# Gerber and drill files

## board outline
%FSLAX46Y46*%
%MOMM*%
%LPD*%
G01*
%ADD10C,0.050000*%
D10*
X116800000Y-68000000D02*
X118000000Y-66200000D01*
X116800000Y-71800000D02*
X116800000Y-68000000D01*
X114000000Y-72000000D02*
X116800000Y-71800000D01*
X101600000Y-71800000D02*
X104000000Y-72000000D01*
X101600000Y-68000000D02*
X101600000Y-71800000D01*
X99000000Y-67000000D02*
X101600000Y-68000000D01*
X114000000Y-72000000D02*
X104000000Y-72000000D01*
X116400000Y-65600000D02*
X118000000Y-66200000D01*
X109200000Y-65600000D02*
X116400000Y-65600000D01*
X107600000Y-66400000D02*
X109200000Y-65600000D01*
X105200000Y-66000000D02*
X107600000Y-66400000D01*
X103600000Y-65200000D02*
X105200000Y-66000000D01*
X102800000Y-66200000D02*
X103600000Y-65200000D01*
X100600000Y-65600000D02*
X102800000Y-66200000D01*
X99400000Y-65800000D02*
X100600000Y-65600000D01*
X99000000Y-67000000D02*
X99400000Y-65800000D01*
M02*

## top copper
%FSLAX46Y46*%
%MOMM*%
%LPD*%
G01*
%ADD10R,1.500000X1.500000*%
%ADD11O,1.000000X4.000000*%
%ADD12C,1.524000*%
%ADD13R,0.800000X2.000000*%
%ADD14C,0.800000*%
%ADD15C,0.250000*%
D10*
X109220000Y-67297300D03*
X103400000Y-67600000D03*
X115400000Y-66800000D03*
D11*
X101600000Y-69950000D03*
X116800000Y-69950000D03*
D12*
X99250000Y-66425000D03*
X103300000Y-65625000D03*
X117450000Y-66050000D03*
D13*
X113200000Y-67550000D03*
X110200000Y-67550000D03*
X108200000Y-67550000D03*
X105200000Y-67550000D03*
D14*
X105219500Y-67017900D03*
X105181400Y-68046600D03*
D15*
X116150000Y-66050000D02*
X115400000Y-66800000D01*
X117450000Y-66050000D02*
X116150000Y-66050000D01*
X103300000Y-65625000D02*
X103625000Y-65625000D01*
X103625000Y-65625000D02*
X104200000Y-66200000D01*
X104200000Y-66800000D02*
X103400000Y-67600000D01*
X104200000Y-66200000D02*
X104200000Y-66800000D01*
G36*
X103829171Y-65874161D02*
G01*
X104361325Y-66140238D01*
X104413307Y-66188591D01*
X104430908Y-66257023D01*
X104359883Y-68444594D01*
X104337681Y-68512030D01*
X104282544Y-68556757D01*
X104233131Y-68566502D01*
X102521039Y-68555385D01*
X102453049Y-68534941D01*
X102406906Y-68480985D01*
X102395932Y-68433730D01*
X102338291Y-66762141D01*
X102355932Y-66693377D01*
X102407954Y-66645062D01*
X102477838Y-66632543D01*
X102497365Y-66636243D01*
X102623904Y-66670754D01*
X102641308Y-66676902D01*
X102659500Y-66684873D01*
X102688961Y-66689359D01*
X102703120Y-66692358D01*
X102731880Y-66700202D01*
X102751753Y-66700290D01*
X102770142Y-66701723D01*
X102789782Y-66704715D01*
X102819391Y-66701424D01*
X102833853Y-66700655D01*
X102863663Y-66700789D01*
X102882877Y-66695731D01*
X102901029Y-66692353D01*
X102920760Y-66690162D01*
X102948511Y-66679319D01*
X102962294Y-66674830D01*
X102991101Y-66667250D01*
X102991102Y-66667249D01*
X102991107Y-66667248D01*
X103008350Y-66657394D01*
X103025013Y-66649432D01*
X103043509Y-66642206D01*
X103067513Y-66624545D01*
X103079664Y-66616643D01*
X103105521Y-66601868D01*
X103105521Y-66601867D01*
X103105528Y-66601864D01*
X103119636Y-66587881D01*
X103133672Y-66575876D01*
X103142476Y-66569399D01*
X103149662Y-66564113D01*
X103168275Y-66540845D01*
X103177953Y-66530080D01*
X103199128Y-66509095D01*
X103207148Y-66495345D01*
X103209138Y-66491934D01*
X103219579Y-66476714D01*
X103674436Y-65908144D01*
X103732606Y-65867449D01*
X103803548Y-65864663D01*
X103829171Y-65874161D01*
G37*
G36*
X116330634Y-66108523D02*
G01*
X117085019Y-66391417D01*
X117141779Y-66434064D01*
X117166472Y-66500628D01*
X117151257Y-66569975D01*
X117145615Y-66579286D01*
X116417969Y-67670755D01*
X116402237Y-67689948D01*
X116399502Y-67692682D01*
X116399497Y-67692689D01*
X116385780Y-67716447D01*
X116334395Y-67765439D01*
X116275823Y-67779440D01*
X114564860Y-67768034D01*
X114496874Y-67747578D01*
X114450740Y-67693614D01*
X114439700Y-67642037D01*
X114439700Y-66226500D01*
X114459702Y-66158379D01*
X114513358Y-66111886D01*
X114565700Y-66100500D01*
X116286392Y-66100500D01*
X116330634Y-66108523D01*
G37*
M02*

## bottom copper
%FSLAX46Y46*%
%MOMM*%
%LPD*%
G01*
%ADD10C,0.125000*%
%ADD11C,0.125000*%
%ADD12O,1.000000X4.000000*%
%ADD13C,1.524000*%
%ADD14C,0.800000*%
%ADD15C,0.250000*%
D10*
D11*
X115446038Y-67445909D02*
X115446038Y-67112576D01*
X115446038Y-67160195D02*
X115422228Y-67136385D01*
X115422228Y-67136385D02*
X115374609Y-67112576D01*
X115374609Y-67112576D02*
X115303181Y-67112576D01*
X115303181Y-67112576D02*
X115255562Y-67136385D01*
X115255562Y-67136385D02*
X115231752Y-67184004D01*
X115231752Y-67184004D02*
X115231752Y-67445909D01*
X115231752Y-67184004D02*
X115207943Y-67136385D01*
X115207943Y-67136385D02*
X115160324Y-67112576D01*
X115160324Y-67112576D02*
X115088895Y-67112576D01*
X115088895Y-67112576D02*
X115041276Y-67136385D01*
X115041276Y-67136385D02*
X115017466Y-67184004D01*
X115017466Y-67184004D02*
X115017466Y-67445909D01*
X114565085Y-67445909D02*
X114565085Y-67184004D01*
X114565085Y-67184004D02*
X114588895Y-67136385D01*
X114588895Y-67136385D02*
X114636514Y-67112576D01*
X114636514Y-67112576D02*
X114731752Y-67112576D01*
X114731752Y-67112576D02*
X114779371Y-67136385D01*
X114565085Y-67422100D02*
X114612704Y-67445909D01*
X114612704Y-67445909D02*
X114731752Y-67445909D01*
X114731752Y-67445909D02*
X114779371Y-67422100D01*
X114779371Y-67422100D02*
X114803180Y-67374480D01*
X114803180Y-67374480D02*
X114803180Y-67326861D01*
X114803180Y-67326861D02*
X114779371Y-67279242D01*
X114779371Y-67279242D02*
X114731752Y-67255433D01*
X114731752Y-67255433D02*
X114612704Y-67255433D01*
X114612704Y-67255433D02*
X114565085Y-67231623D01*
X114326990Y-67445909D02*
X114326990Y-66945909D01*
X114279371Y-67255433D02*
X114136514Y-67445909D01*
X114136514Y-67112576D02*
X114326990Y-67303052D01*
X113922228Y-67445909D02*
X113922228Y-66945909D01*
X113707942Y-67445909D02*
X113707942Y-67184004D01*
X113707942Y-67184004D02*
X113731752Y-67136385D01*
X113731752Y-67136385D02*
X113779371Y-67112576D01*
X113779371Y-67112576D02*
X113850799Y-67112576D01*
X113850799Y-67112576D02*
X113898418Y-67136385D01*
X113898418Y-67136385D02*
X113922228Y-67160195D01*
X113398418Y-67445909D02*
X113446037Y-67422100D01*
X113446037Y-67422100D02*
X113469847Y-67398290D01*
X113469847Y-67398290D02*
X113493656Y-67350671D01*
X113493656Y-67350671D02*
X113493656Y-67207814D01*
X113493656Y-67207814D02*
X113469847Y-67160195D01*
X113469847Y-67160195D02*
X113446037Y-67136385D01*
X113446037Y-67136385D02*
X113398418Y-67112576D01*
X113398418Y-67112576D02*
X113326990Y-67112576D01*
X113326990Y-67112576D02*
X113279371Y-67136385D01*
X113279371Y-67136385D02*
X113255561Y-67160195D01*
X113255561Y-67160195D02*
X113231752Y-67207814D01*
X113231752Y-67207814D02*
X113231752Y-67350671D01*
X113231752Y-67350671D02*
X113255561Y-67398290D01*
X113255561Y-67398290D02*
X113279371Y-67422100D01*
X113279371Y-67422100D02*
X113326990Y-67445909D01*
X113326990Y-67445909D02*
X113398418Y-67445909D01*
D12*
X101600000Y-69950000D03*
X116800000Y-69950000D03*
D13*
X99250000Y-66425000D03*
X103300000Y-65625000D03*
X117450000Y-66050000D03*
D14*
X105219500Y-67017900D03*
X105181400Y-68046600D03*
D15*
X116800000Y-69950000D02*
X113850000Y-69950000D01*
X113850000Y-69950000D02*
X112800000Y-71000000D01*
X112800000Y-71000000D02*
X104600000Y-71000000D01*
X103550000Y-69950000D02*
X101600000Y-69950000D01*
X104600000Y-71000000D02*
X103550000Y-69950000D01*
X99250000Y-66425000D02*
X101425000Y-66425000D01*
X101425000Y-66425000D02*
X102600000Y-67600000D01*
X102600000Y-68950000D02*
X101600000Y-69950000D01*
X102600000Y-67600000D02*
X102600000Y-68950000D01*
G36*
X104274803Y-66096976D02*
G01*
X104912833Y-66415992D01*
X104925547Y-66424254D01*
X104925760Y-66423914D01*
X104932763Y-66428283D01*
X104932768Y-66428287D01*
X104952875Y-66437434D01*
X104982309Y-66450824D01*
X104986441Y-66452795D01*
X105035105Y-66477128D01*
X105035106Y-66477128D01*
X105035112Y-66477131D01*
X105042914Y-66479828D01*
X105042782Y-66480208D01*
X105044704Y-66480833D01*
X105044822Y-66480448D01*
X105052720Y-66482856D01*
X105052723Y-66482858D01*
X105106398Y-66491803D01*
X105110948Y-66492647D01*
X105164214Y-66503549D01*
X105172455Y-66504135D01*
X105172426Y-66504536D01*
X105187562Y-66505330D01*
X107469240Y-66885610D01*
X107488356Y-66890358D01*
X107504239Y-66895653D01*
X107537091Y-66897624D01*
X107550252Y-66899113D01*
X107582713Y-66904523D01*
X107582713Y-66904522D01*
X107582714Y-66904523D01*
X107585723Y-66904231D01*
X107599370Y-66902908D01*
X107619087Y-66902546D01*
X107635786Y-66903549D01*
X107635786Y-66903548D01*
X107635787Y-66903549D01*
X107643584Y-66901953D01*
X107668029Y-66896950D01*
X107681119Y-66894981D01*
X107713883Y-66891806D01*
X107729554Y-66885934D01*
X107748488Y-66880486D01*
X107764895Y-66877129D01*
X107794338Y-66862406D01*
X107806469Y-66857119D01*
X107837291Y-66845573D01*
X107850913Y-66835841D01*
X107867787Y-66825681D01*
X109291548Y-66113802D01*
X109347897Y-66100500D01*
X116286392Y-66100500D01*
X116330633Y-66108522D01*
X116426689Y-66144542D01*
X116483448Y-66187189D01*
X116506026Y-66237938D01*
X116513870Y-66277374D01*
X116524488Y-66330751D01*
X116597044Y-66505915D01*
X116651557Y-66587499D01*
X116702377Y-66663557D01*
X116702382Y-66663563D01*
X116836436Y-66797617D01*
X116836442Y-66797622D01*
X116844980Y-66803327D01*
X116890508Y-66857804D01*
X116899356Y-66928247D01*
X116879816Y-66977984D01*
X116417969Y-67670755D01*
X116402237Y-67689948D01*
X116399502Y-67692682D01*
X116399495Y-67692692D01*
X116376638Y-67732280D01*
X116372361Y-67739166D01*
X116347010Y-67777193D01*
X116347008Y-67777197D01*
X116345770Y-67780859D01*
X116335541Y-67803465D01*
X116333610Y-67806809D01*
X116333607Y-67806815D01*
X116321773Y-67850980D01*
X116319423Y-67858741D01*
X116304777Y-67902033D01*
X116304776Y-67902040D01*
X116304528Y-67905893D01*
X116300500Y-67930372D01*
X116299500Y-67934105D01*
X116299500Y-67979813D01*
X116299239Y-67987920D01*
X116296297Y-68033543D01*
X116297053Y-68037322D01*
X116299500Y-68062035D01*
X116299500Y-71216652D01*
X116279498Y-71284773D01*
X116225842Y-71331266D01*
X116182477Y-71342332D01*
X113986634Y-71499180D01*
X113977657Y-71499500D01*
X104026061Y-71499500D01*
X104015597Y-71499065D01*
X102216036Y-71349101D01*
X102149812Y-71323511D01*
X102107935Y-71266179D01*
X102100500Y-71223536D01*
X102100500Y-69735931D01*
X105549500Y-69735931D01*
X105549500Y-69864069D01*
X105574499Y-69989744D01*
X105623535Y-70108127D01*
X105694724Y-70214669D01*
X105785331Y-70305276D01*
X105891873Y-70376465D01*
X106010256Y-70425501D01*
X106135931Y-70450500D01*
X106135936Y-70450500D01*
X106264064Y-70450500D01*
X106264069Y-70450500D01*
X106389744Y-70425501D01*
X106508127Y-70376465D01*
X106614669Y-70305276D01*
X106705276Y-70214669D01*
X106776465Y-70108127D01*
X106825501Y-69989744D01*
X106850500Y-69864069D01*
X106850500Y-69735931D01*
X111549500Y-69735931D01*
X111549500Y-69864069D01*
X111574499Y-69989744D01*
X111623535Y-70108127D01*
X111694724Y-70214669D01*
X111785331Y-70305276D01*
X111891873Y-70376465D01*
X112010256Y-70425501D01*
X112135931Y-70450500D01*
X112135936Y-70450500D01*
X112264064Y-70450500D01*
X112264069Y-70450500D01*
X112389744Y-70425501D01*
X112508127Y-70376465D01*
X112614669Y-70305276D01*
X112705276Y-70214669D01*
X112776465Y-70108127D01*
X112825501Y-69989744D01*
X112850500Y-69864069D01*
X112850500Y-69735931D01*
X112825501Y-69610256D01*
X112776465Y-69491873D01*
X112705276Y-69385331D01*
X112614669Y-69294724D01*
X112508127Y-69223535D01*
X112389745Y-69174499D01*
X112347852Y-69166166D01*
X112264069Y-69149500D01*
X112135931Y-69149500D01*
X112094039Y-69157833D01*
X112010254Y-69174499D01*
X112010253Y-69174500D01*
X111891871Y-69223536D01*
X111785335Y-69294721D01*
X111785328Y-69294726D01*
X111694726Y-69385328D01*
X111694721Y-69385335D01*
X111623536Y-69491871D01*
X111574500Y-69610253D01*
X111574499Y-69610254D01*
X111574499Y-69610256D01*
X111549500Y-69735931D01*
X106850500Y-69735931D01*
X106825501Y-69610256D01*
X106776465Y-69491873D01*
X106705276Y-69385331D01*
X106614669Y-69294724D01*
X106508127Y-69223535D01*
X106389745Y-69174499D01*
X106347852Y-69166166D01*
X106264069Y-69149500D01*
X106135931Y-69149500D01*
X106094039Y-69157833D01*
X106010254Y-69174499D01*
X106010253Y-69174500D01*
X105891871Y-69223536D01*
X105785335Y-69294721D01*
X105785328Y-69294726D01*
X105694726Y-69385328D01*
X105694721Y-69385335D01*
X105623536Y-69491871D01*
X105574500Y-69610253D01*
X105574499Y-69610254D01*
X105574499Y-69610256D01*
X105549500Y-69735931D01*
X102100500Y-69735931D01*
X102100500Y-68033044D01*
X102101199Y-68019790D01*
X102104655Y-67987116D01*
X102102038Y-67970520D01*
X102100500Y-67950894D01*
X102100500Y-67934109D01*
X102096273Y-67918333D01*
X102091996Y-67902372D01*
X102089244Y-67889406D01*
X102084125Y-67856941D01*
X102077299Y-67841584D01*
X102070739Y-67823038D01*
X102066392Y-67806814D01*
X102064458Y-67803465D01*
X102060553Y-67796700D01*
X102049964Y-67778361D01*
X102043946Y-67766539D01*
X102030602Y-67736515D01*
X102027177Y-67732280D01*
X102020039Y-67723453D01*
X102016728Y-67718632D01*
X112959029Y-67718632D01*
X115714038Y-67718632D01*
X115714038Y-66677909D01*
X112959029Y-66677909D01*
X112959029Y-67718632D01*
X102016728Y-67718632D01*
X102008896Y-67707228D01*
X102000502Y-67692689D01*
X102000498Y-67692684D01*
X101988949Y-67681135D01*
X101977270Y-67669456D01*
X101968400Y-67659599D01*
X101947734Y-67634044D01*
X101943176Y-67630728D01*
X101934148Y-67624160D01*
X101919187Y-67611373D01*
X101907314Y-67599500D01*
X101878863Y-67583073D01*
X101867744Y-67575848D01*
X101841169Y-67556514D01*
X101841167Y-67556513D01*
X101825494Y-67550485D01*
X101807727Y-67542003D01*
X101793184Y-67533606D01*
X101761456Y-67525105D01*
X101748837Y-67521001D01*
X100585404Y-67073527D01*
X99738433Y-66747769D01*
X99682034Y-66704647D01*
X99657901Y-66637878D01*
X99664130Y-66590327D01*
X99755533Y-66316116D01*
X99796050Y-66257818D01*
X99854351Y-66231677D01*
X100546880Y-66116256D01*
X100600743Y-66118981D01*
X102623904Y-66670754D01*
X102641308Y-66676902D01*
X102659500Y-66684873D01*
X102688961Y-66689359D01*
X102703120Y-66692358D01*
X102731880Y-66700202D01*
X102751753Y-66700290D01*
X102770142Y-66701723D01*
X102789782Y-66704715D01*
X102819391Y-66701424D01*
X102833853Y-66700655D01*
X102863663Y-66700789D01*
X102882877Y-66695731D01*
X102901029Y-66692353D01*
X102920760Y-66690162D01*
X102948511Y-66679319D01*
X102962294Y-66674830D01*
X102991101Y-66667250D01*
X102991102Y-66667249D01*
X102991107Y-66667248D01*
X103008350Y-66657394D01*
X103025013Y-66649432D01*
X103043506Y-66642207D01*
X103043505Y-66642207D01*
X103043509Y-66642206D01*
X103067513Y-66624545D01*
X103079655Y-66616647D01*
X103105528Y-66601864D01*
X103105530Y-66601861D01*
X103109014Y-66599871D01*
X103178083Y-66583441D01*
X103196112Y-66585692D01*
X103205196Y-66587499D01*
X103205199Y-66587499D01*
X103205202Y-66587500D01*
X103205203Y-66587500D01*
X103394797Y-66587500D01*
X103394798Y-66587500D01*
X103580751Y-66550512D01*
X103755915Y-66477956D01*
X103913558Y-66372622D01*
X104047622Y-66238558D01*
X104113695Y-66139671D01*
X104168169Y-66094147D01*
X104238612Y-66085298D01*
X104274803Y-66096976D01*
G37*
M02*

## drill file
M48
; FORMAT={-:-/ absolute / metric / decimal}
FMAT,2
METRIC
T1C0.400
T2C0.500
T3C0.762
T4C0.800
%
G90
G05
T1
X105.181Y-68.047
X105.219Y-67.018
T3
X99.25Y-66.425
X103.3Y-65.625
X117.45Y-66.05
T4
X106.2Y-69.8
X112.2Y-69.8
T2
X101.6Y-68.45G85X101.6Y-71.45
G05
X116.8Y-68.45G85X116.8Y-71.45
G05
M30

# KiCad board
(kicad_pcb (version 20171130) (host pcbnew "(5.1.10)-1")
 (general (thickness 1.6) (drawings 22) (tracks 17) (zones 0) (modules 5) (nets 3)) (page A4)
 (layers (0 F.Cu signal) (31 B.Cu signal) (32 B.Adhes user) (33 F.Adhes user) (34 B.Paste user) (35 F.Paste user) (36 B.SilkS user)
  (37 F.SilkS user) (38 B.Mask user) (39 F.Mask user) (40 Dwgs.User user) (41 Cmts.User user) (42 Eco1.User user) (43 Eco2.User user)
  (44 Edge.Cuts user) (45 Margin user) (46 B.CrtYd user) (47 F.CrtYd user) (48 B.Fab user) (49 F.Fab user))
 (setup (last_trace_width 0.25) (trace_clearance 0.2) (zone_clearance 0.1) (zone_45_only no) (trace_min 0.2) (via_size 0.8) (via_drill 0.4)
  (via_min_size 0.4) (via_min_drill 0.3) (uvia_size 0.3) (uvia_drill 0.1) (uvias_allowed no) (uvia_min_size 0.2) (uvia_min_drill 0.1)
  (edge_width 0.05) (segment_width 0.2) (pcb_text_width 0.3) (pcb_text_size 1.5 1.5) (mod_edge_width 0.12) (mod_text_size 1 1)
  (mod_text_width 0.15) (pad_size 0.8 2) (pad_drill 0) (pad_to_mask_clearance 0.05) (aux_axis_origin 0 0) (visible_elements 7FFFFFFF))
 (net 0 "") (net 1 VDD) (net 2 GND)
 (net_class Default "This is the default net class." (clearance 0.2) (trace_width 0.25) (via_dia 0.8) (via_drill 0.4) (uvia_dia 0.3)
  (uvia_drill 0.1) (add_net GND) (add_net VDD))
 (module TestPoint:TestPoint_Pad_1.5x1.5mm (layer F.Cu) (at 109.22 67.2973)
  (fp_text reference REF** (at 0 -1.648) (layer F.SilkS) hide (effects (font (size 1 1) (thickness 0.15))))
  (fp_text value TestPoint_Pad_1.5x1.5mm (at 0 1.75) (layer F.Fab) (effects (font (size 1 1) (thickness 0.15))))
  (pad 1 smd rect (at 0 0) (size 1.5 1.5) (layers F.Cu F.Mask)))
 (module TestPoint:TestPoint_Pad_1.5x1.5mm (layer F.Cu) (at 103.4 67.6)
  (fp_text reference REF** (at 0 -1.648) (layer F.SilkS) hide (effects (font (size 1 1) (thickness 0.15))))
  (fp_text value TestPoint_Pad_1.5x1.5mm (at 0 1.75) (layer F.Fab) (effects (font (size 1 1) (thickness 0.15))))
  (pad 1 smd rect (at 0 0) (size 1.5 1.5) (layers F.Cu F.Mask) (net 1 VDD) (zone_connect 2)))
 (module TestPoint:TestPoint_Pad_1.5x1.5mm (layer F.Cu) (at 115.4 66.8)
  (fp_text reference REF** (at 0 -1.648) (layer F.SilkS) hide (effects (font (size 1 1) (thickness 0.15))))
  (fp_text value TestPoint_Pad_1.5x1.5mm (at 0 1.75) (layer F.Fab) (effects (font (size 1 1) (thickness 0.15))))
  (pad 1 smd rect (at 0 0) (size 1.5 1.5) (layers F.Cu F.Mask) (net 1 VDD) (zone_connect 2)))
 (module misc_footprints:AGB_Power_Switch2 (layer F.Cu) (at 108.4 70.2)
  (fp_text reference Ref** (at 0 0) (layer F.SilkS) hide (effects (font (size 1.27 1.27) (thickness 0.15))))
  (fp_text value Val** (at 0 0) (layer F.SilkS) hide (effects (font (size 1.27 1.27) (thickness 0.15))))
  (pad 3 thru_hole oval (at -6.8 -0.25) (size 1 4) (drill oval 0.5 3.5) (layers *.Cu *.Mask) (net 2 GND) (zone_connect 2))
  (pad 3 thru_hole oval (at 8.4 -0.25) (size 1 4) (drill oval 0.5 3.5) (layers *.Cu *.Mask) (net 2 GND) (zone_connect 2))
  (pad 3 thru_hole circle (at -9.15 -3.775) (size 1.524 1.524) (drill 0.762) (layers *.Cu *.Mask) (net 2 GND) (zone_connect 2))
  (pad 2 thru_hole circle (at -5.1 -4.575) (size 1.524 1.524) (drill 0.762) (layers *.Cu *.Mask) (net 1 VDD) (zone_connect 2))
  (pad 1 thru_hole circle (at 9.05 -4.15) (size 1.524 1.524) (drill 0.762) (layers *.Cu *.Mask) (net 1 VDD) (zone_connect 2)))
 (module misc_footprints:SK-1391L (layer F.Cu) (at 109.2 69.8)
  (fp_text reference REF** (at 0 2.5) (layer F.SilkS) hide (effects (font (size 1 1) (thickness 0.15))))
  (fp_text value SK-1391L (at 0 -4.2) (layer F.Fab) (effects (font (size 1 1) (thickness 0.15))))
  (pad "" np_thru_hole circle (at 3 0) (size 0.8 0.8) (drill 0.8) (layers *.Cu *.Mask))
  (pad "" np_thru_hole circle (at -3 0) (size 0.8 0.8) (drill 0.8) (layers *.Cu *.Mask))
  (pad 4 smd rect (at 4 -2.25) (size 0.8 2) (layers F.Cu F.Paste F.Mask))
  (pad 3 smd rect (at 1 -2.25) (size 0.8 2) (layers F.Cu F.Paste F.Mask))
  (pad 2 smd rect (at -1 -2.25) (size 0.8 2) (layers F.Cu F.Paste F.Mask))
  (pad 1 smd rect (at -4 -2.25) (size 0.8 2) (layers F.Cu F.Paste F.Mask) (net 2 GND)))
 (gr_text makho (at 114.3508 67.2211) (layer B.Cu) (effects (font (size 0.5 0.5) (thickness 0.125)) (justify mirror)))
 (gr_line (start 116.8 68) (end 118 66.2) (layer Edge.Cuts) (width 0.05))
 (gr_line (start 116.8 71.8) (end 116.8 68) (layer Edge.Cuts) (width 0.05))
 (gr_line (start 114 72) (end 116.8 71.8) (layer Edge.Cuts) (width 0.05))
 (gr_line (start 101.6 71.8) (end 104 72) (layer Edge.Cuts) (width 0.05))
 (gr_line (start 101.6 68) (end 101.6 71.8) (layer Edge.Cuts) (width 0.05))
 (gr_line (start 99 67) (end 101.6 68) (layer Edge.Cuts) (width 0.05))
 (gr_line (start 114 72) (end 104 72) (layer Edge.Cuts) (width 0.05))
 (gr_line (start 116.4 65.6) (end 118 66.2) (layer Edge.Cuts) (width 0.05))
 (gr_line (start 109.2 65.6) (end 116.4 65.6) (layer Edge.Cuts) (width 0.05))
 (gr_line (start 107.6 66.4) (end 109.2 65.6) (layer Edge.Cuts) (width 0.05))
 (gr_line (start 105.2 66) (end 107.6 66.4) (layer Edge.Cuts) (width 0.05))
 (gr_line (start 103.6 65.2) (end 105.2 66) (layer Edge.Cuts) (width 0.05))
 (gr_line (start 102.8 66.2) (end 103.6 65.2) (layer Edge.Cuts) (width 0.05))
 (gr_line (start 100.6 65.6) (end 102.8 66.2) (layer Edge.Cuts) (width 0.05))
 (gr_line (start 99.4 65.8) (end 100.6 65.6) (layer Edge.Cuts) (width 0.05))
 (gr_line (start 99 67) (end 99.4 65.8) (layer Edge.Cuts) (width 0.05))
 (via (at 105.2195 67.0179) (size 0.8) (drill 0.4) (layers F.Cu B.Cu) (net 2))
 (via (at 105.1814 68.0466) (size 0.8) (drill 0.4) (layers F.Cu B.Cu) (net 2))
 (segment (start 116.8 69.95) (end 113.85 69.95) (width 0.25) (layer B.Cu) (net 2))
 (segment (start 113.85 69.95) (end 112.8 71) (width 0.25) (layer B.Cu) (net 2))
 (segment (start 112.8 71) (end 104.6 71) (width 0.25) (layer B.Cu) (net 2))
 (segment (start 103.55 69.95) (end 101.6 69.95) (width 0.25) (layer B.Cu) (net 2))
 (segment (start 104.6 71) (end 103.55 69.95) (width 0.25) (layer B.Cu) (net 2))
 (segment (start 99.25 66.425) (end 101.425 66.425) (width 0.25) (layer B.Cu) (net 2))
 (segment (start 101.425 66.425) (end 102.6 67.6) (width 0.25) (layer B.Cu) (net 2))
 (segment (start 102.6 68.95) (end 101.6 69.95) (width 0.25) (layer B.Cu) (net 2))
 (segment (start 102.6 67.6) (end 102.6 68.95) (width 0.25) (layer B.Cu) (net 2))
 (segment (start 116.15 66.05) (end 115.4 66.8) (width 0.25) (layer F.Cu) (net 1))
 (segment (start 117.45 66.05) (end 116.15 66.05) (width 0.25) (layer F.Cu) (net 1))
 (segment (start 103.3 65.625) (end 103.625 65.625) (width 0.25) (layer F.Cu) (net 1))
 (segment (start 103.625 65.625) (end 104.2 66.2) (width 0.25) (layer F.Cu) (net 1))
 (segment (start 104.2 66.8) (end 103.4 67.6) (width 0.25) (layer F.Cu) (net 1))
 (segment (start 104.2 66.2) (end 104.2 66.8) (width 0.25) (layer F.Cu) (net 1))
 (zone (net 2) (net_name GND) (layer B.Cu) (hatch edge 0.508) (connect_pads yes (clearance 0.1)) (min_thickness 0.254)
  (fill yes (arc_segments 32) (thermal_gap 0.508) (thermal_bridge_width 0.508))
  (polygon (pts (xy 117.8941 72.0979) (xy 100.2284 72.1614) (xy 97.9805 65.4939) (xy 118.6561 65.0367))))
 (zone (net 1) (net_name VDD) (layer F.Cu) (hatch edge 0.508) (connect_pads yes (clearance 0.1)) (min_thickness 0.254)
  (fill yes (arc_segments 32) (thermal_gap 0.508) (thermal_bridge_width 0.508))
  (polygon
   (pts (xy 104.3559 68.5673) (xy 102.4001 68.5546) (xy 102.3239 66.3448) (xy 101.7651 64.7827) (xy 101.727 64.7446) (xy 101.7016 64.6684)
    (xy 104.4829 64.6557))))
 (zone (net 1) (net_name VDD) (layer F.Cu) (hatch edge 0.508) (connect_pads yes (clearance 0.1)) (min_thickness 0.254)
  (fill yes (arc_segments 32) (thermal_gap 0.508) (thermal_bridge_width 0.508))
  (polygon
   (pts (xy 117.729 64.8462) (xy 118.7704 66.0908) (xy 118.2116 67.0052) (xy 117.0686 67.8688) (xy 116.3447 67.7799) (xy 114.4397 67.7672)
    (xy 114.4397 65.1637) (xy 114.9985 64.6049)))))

